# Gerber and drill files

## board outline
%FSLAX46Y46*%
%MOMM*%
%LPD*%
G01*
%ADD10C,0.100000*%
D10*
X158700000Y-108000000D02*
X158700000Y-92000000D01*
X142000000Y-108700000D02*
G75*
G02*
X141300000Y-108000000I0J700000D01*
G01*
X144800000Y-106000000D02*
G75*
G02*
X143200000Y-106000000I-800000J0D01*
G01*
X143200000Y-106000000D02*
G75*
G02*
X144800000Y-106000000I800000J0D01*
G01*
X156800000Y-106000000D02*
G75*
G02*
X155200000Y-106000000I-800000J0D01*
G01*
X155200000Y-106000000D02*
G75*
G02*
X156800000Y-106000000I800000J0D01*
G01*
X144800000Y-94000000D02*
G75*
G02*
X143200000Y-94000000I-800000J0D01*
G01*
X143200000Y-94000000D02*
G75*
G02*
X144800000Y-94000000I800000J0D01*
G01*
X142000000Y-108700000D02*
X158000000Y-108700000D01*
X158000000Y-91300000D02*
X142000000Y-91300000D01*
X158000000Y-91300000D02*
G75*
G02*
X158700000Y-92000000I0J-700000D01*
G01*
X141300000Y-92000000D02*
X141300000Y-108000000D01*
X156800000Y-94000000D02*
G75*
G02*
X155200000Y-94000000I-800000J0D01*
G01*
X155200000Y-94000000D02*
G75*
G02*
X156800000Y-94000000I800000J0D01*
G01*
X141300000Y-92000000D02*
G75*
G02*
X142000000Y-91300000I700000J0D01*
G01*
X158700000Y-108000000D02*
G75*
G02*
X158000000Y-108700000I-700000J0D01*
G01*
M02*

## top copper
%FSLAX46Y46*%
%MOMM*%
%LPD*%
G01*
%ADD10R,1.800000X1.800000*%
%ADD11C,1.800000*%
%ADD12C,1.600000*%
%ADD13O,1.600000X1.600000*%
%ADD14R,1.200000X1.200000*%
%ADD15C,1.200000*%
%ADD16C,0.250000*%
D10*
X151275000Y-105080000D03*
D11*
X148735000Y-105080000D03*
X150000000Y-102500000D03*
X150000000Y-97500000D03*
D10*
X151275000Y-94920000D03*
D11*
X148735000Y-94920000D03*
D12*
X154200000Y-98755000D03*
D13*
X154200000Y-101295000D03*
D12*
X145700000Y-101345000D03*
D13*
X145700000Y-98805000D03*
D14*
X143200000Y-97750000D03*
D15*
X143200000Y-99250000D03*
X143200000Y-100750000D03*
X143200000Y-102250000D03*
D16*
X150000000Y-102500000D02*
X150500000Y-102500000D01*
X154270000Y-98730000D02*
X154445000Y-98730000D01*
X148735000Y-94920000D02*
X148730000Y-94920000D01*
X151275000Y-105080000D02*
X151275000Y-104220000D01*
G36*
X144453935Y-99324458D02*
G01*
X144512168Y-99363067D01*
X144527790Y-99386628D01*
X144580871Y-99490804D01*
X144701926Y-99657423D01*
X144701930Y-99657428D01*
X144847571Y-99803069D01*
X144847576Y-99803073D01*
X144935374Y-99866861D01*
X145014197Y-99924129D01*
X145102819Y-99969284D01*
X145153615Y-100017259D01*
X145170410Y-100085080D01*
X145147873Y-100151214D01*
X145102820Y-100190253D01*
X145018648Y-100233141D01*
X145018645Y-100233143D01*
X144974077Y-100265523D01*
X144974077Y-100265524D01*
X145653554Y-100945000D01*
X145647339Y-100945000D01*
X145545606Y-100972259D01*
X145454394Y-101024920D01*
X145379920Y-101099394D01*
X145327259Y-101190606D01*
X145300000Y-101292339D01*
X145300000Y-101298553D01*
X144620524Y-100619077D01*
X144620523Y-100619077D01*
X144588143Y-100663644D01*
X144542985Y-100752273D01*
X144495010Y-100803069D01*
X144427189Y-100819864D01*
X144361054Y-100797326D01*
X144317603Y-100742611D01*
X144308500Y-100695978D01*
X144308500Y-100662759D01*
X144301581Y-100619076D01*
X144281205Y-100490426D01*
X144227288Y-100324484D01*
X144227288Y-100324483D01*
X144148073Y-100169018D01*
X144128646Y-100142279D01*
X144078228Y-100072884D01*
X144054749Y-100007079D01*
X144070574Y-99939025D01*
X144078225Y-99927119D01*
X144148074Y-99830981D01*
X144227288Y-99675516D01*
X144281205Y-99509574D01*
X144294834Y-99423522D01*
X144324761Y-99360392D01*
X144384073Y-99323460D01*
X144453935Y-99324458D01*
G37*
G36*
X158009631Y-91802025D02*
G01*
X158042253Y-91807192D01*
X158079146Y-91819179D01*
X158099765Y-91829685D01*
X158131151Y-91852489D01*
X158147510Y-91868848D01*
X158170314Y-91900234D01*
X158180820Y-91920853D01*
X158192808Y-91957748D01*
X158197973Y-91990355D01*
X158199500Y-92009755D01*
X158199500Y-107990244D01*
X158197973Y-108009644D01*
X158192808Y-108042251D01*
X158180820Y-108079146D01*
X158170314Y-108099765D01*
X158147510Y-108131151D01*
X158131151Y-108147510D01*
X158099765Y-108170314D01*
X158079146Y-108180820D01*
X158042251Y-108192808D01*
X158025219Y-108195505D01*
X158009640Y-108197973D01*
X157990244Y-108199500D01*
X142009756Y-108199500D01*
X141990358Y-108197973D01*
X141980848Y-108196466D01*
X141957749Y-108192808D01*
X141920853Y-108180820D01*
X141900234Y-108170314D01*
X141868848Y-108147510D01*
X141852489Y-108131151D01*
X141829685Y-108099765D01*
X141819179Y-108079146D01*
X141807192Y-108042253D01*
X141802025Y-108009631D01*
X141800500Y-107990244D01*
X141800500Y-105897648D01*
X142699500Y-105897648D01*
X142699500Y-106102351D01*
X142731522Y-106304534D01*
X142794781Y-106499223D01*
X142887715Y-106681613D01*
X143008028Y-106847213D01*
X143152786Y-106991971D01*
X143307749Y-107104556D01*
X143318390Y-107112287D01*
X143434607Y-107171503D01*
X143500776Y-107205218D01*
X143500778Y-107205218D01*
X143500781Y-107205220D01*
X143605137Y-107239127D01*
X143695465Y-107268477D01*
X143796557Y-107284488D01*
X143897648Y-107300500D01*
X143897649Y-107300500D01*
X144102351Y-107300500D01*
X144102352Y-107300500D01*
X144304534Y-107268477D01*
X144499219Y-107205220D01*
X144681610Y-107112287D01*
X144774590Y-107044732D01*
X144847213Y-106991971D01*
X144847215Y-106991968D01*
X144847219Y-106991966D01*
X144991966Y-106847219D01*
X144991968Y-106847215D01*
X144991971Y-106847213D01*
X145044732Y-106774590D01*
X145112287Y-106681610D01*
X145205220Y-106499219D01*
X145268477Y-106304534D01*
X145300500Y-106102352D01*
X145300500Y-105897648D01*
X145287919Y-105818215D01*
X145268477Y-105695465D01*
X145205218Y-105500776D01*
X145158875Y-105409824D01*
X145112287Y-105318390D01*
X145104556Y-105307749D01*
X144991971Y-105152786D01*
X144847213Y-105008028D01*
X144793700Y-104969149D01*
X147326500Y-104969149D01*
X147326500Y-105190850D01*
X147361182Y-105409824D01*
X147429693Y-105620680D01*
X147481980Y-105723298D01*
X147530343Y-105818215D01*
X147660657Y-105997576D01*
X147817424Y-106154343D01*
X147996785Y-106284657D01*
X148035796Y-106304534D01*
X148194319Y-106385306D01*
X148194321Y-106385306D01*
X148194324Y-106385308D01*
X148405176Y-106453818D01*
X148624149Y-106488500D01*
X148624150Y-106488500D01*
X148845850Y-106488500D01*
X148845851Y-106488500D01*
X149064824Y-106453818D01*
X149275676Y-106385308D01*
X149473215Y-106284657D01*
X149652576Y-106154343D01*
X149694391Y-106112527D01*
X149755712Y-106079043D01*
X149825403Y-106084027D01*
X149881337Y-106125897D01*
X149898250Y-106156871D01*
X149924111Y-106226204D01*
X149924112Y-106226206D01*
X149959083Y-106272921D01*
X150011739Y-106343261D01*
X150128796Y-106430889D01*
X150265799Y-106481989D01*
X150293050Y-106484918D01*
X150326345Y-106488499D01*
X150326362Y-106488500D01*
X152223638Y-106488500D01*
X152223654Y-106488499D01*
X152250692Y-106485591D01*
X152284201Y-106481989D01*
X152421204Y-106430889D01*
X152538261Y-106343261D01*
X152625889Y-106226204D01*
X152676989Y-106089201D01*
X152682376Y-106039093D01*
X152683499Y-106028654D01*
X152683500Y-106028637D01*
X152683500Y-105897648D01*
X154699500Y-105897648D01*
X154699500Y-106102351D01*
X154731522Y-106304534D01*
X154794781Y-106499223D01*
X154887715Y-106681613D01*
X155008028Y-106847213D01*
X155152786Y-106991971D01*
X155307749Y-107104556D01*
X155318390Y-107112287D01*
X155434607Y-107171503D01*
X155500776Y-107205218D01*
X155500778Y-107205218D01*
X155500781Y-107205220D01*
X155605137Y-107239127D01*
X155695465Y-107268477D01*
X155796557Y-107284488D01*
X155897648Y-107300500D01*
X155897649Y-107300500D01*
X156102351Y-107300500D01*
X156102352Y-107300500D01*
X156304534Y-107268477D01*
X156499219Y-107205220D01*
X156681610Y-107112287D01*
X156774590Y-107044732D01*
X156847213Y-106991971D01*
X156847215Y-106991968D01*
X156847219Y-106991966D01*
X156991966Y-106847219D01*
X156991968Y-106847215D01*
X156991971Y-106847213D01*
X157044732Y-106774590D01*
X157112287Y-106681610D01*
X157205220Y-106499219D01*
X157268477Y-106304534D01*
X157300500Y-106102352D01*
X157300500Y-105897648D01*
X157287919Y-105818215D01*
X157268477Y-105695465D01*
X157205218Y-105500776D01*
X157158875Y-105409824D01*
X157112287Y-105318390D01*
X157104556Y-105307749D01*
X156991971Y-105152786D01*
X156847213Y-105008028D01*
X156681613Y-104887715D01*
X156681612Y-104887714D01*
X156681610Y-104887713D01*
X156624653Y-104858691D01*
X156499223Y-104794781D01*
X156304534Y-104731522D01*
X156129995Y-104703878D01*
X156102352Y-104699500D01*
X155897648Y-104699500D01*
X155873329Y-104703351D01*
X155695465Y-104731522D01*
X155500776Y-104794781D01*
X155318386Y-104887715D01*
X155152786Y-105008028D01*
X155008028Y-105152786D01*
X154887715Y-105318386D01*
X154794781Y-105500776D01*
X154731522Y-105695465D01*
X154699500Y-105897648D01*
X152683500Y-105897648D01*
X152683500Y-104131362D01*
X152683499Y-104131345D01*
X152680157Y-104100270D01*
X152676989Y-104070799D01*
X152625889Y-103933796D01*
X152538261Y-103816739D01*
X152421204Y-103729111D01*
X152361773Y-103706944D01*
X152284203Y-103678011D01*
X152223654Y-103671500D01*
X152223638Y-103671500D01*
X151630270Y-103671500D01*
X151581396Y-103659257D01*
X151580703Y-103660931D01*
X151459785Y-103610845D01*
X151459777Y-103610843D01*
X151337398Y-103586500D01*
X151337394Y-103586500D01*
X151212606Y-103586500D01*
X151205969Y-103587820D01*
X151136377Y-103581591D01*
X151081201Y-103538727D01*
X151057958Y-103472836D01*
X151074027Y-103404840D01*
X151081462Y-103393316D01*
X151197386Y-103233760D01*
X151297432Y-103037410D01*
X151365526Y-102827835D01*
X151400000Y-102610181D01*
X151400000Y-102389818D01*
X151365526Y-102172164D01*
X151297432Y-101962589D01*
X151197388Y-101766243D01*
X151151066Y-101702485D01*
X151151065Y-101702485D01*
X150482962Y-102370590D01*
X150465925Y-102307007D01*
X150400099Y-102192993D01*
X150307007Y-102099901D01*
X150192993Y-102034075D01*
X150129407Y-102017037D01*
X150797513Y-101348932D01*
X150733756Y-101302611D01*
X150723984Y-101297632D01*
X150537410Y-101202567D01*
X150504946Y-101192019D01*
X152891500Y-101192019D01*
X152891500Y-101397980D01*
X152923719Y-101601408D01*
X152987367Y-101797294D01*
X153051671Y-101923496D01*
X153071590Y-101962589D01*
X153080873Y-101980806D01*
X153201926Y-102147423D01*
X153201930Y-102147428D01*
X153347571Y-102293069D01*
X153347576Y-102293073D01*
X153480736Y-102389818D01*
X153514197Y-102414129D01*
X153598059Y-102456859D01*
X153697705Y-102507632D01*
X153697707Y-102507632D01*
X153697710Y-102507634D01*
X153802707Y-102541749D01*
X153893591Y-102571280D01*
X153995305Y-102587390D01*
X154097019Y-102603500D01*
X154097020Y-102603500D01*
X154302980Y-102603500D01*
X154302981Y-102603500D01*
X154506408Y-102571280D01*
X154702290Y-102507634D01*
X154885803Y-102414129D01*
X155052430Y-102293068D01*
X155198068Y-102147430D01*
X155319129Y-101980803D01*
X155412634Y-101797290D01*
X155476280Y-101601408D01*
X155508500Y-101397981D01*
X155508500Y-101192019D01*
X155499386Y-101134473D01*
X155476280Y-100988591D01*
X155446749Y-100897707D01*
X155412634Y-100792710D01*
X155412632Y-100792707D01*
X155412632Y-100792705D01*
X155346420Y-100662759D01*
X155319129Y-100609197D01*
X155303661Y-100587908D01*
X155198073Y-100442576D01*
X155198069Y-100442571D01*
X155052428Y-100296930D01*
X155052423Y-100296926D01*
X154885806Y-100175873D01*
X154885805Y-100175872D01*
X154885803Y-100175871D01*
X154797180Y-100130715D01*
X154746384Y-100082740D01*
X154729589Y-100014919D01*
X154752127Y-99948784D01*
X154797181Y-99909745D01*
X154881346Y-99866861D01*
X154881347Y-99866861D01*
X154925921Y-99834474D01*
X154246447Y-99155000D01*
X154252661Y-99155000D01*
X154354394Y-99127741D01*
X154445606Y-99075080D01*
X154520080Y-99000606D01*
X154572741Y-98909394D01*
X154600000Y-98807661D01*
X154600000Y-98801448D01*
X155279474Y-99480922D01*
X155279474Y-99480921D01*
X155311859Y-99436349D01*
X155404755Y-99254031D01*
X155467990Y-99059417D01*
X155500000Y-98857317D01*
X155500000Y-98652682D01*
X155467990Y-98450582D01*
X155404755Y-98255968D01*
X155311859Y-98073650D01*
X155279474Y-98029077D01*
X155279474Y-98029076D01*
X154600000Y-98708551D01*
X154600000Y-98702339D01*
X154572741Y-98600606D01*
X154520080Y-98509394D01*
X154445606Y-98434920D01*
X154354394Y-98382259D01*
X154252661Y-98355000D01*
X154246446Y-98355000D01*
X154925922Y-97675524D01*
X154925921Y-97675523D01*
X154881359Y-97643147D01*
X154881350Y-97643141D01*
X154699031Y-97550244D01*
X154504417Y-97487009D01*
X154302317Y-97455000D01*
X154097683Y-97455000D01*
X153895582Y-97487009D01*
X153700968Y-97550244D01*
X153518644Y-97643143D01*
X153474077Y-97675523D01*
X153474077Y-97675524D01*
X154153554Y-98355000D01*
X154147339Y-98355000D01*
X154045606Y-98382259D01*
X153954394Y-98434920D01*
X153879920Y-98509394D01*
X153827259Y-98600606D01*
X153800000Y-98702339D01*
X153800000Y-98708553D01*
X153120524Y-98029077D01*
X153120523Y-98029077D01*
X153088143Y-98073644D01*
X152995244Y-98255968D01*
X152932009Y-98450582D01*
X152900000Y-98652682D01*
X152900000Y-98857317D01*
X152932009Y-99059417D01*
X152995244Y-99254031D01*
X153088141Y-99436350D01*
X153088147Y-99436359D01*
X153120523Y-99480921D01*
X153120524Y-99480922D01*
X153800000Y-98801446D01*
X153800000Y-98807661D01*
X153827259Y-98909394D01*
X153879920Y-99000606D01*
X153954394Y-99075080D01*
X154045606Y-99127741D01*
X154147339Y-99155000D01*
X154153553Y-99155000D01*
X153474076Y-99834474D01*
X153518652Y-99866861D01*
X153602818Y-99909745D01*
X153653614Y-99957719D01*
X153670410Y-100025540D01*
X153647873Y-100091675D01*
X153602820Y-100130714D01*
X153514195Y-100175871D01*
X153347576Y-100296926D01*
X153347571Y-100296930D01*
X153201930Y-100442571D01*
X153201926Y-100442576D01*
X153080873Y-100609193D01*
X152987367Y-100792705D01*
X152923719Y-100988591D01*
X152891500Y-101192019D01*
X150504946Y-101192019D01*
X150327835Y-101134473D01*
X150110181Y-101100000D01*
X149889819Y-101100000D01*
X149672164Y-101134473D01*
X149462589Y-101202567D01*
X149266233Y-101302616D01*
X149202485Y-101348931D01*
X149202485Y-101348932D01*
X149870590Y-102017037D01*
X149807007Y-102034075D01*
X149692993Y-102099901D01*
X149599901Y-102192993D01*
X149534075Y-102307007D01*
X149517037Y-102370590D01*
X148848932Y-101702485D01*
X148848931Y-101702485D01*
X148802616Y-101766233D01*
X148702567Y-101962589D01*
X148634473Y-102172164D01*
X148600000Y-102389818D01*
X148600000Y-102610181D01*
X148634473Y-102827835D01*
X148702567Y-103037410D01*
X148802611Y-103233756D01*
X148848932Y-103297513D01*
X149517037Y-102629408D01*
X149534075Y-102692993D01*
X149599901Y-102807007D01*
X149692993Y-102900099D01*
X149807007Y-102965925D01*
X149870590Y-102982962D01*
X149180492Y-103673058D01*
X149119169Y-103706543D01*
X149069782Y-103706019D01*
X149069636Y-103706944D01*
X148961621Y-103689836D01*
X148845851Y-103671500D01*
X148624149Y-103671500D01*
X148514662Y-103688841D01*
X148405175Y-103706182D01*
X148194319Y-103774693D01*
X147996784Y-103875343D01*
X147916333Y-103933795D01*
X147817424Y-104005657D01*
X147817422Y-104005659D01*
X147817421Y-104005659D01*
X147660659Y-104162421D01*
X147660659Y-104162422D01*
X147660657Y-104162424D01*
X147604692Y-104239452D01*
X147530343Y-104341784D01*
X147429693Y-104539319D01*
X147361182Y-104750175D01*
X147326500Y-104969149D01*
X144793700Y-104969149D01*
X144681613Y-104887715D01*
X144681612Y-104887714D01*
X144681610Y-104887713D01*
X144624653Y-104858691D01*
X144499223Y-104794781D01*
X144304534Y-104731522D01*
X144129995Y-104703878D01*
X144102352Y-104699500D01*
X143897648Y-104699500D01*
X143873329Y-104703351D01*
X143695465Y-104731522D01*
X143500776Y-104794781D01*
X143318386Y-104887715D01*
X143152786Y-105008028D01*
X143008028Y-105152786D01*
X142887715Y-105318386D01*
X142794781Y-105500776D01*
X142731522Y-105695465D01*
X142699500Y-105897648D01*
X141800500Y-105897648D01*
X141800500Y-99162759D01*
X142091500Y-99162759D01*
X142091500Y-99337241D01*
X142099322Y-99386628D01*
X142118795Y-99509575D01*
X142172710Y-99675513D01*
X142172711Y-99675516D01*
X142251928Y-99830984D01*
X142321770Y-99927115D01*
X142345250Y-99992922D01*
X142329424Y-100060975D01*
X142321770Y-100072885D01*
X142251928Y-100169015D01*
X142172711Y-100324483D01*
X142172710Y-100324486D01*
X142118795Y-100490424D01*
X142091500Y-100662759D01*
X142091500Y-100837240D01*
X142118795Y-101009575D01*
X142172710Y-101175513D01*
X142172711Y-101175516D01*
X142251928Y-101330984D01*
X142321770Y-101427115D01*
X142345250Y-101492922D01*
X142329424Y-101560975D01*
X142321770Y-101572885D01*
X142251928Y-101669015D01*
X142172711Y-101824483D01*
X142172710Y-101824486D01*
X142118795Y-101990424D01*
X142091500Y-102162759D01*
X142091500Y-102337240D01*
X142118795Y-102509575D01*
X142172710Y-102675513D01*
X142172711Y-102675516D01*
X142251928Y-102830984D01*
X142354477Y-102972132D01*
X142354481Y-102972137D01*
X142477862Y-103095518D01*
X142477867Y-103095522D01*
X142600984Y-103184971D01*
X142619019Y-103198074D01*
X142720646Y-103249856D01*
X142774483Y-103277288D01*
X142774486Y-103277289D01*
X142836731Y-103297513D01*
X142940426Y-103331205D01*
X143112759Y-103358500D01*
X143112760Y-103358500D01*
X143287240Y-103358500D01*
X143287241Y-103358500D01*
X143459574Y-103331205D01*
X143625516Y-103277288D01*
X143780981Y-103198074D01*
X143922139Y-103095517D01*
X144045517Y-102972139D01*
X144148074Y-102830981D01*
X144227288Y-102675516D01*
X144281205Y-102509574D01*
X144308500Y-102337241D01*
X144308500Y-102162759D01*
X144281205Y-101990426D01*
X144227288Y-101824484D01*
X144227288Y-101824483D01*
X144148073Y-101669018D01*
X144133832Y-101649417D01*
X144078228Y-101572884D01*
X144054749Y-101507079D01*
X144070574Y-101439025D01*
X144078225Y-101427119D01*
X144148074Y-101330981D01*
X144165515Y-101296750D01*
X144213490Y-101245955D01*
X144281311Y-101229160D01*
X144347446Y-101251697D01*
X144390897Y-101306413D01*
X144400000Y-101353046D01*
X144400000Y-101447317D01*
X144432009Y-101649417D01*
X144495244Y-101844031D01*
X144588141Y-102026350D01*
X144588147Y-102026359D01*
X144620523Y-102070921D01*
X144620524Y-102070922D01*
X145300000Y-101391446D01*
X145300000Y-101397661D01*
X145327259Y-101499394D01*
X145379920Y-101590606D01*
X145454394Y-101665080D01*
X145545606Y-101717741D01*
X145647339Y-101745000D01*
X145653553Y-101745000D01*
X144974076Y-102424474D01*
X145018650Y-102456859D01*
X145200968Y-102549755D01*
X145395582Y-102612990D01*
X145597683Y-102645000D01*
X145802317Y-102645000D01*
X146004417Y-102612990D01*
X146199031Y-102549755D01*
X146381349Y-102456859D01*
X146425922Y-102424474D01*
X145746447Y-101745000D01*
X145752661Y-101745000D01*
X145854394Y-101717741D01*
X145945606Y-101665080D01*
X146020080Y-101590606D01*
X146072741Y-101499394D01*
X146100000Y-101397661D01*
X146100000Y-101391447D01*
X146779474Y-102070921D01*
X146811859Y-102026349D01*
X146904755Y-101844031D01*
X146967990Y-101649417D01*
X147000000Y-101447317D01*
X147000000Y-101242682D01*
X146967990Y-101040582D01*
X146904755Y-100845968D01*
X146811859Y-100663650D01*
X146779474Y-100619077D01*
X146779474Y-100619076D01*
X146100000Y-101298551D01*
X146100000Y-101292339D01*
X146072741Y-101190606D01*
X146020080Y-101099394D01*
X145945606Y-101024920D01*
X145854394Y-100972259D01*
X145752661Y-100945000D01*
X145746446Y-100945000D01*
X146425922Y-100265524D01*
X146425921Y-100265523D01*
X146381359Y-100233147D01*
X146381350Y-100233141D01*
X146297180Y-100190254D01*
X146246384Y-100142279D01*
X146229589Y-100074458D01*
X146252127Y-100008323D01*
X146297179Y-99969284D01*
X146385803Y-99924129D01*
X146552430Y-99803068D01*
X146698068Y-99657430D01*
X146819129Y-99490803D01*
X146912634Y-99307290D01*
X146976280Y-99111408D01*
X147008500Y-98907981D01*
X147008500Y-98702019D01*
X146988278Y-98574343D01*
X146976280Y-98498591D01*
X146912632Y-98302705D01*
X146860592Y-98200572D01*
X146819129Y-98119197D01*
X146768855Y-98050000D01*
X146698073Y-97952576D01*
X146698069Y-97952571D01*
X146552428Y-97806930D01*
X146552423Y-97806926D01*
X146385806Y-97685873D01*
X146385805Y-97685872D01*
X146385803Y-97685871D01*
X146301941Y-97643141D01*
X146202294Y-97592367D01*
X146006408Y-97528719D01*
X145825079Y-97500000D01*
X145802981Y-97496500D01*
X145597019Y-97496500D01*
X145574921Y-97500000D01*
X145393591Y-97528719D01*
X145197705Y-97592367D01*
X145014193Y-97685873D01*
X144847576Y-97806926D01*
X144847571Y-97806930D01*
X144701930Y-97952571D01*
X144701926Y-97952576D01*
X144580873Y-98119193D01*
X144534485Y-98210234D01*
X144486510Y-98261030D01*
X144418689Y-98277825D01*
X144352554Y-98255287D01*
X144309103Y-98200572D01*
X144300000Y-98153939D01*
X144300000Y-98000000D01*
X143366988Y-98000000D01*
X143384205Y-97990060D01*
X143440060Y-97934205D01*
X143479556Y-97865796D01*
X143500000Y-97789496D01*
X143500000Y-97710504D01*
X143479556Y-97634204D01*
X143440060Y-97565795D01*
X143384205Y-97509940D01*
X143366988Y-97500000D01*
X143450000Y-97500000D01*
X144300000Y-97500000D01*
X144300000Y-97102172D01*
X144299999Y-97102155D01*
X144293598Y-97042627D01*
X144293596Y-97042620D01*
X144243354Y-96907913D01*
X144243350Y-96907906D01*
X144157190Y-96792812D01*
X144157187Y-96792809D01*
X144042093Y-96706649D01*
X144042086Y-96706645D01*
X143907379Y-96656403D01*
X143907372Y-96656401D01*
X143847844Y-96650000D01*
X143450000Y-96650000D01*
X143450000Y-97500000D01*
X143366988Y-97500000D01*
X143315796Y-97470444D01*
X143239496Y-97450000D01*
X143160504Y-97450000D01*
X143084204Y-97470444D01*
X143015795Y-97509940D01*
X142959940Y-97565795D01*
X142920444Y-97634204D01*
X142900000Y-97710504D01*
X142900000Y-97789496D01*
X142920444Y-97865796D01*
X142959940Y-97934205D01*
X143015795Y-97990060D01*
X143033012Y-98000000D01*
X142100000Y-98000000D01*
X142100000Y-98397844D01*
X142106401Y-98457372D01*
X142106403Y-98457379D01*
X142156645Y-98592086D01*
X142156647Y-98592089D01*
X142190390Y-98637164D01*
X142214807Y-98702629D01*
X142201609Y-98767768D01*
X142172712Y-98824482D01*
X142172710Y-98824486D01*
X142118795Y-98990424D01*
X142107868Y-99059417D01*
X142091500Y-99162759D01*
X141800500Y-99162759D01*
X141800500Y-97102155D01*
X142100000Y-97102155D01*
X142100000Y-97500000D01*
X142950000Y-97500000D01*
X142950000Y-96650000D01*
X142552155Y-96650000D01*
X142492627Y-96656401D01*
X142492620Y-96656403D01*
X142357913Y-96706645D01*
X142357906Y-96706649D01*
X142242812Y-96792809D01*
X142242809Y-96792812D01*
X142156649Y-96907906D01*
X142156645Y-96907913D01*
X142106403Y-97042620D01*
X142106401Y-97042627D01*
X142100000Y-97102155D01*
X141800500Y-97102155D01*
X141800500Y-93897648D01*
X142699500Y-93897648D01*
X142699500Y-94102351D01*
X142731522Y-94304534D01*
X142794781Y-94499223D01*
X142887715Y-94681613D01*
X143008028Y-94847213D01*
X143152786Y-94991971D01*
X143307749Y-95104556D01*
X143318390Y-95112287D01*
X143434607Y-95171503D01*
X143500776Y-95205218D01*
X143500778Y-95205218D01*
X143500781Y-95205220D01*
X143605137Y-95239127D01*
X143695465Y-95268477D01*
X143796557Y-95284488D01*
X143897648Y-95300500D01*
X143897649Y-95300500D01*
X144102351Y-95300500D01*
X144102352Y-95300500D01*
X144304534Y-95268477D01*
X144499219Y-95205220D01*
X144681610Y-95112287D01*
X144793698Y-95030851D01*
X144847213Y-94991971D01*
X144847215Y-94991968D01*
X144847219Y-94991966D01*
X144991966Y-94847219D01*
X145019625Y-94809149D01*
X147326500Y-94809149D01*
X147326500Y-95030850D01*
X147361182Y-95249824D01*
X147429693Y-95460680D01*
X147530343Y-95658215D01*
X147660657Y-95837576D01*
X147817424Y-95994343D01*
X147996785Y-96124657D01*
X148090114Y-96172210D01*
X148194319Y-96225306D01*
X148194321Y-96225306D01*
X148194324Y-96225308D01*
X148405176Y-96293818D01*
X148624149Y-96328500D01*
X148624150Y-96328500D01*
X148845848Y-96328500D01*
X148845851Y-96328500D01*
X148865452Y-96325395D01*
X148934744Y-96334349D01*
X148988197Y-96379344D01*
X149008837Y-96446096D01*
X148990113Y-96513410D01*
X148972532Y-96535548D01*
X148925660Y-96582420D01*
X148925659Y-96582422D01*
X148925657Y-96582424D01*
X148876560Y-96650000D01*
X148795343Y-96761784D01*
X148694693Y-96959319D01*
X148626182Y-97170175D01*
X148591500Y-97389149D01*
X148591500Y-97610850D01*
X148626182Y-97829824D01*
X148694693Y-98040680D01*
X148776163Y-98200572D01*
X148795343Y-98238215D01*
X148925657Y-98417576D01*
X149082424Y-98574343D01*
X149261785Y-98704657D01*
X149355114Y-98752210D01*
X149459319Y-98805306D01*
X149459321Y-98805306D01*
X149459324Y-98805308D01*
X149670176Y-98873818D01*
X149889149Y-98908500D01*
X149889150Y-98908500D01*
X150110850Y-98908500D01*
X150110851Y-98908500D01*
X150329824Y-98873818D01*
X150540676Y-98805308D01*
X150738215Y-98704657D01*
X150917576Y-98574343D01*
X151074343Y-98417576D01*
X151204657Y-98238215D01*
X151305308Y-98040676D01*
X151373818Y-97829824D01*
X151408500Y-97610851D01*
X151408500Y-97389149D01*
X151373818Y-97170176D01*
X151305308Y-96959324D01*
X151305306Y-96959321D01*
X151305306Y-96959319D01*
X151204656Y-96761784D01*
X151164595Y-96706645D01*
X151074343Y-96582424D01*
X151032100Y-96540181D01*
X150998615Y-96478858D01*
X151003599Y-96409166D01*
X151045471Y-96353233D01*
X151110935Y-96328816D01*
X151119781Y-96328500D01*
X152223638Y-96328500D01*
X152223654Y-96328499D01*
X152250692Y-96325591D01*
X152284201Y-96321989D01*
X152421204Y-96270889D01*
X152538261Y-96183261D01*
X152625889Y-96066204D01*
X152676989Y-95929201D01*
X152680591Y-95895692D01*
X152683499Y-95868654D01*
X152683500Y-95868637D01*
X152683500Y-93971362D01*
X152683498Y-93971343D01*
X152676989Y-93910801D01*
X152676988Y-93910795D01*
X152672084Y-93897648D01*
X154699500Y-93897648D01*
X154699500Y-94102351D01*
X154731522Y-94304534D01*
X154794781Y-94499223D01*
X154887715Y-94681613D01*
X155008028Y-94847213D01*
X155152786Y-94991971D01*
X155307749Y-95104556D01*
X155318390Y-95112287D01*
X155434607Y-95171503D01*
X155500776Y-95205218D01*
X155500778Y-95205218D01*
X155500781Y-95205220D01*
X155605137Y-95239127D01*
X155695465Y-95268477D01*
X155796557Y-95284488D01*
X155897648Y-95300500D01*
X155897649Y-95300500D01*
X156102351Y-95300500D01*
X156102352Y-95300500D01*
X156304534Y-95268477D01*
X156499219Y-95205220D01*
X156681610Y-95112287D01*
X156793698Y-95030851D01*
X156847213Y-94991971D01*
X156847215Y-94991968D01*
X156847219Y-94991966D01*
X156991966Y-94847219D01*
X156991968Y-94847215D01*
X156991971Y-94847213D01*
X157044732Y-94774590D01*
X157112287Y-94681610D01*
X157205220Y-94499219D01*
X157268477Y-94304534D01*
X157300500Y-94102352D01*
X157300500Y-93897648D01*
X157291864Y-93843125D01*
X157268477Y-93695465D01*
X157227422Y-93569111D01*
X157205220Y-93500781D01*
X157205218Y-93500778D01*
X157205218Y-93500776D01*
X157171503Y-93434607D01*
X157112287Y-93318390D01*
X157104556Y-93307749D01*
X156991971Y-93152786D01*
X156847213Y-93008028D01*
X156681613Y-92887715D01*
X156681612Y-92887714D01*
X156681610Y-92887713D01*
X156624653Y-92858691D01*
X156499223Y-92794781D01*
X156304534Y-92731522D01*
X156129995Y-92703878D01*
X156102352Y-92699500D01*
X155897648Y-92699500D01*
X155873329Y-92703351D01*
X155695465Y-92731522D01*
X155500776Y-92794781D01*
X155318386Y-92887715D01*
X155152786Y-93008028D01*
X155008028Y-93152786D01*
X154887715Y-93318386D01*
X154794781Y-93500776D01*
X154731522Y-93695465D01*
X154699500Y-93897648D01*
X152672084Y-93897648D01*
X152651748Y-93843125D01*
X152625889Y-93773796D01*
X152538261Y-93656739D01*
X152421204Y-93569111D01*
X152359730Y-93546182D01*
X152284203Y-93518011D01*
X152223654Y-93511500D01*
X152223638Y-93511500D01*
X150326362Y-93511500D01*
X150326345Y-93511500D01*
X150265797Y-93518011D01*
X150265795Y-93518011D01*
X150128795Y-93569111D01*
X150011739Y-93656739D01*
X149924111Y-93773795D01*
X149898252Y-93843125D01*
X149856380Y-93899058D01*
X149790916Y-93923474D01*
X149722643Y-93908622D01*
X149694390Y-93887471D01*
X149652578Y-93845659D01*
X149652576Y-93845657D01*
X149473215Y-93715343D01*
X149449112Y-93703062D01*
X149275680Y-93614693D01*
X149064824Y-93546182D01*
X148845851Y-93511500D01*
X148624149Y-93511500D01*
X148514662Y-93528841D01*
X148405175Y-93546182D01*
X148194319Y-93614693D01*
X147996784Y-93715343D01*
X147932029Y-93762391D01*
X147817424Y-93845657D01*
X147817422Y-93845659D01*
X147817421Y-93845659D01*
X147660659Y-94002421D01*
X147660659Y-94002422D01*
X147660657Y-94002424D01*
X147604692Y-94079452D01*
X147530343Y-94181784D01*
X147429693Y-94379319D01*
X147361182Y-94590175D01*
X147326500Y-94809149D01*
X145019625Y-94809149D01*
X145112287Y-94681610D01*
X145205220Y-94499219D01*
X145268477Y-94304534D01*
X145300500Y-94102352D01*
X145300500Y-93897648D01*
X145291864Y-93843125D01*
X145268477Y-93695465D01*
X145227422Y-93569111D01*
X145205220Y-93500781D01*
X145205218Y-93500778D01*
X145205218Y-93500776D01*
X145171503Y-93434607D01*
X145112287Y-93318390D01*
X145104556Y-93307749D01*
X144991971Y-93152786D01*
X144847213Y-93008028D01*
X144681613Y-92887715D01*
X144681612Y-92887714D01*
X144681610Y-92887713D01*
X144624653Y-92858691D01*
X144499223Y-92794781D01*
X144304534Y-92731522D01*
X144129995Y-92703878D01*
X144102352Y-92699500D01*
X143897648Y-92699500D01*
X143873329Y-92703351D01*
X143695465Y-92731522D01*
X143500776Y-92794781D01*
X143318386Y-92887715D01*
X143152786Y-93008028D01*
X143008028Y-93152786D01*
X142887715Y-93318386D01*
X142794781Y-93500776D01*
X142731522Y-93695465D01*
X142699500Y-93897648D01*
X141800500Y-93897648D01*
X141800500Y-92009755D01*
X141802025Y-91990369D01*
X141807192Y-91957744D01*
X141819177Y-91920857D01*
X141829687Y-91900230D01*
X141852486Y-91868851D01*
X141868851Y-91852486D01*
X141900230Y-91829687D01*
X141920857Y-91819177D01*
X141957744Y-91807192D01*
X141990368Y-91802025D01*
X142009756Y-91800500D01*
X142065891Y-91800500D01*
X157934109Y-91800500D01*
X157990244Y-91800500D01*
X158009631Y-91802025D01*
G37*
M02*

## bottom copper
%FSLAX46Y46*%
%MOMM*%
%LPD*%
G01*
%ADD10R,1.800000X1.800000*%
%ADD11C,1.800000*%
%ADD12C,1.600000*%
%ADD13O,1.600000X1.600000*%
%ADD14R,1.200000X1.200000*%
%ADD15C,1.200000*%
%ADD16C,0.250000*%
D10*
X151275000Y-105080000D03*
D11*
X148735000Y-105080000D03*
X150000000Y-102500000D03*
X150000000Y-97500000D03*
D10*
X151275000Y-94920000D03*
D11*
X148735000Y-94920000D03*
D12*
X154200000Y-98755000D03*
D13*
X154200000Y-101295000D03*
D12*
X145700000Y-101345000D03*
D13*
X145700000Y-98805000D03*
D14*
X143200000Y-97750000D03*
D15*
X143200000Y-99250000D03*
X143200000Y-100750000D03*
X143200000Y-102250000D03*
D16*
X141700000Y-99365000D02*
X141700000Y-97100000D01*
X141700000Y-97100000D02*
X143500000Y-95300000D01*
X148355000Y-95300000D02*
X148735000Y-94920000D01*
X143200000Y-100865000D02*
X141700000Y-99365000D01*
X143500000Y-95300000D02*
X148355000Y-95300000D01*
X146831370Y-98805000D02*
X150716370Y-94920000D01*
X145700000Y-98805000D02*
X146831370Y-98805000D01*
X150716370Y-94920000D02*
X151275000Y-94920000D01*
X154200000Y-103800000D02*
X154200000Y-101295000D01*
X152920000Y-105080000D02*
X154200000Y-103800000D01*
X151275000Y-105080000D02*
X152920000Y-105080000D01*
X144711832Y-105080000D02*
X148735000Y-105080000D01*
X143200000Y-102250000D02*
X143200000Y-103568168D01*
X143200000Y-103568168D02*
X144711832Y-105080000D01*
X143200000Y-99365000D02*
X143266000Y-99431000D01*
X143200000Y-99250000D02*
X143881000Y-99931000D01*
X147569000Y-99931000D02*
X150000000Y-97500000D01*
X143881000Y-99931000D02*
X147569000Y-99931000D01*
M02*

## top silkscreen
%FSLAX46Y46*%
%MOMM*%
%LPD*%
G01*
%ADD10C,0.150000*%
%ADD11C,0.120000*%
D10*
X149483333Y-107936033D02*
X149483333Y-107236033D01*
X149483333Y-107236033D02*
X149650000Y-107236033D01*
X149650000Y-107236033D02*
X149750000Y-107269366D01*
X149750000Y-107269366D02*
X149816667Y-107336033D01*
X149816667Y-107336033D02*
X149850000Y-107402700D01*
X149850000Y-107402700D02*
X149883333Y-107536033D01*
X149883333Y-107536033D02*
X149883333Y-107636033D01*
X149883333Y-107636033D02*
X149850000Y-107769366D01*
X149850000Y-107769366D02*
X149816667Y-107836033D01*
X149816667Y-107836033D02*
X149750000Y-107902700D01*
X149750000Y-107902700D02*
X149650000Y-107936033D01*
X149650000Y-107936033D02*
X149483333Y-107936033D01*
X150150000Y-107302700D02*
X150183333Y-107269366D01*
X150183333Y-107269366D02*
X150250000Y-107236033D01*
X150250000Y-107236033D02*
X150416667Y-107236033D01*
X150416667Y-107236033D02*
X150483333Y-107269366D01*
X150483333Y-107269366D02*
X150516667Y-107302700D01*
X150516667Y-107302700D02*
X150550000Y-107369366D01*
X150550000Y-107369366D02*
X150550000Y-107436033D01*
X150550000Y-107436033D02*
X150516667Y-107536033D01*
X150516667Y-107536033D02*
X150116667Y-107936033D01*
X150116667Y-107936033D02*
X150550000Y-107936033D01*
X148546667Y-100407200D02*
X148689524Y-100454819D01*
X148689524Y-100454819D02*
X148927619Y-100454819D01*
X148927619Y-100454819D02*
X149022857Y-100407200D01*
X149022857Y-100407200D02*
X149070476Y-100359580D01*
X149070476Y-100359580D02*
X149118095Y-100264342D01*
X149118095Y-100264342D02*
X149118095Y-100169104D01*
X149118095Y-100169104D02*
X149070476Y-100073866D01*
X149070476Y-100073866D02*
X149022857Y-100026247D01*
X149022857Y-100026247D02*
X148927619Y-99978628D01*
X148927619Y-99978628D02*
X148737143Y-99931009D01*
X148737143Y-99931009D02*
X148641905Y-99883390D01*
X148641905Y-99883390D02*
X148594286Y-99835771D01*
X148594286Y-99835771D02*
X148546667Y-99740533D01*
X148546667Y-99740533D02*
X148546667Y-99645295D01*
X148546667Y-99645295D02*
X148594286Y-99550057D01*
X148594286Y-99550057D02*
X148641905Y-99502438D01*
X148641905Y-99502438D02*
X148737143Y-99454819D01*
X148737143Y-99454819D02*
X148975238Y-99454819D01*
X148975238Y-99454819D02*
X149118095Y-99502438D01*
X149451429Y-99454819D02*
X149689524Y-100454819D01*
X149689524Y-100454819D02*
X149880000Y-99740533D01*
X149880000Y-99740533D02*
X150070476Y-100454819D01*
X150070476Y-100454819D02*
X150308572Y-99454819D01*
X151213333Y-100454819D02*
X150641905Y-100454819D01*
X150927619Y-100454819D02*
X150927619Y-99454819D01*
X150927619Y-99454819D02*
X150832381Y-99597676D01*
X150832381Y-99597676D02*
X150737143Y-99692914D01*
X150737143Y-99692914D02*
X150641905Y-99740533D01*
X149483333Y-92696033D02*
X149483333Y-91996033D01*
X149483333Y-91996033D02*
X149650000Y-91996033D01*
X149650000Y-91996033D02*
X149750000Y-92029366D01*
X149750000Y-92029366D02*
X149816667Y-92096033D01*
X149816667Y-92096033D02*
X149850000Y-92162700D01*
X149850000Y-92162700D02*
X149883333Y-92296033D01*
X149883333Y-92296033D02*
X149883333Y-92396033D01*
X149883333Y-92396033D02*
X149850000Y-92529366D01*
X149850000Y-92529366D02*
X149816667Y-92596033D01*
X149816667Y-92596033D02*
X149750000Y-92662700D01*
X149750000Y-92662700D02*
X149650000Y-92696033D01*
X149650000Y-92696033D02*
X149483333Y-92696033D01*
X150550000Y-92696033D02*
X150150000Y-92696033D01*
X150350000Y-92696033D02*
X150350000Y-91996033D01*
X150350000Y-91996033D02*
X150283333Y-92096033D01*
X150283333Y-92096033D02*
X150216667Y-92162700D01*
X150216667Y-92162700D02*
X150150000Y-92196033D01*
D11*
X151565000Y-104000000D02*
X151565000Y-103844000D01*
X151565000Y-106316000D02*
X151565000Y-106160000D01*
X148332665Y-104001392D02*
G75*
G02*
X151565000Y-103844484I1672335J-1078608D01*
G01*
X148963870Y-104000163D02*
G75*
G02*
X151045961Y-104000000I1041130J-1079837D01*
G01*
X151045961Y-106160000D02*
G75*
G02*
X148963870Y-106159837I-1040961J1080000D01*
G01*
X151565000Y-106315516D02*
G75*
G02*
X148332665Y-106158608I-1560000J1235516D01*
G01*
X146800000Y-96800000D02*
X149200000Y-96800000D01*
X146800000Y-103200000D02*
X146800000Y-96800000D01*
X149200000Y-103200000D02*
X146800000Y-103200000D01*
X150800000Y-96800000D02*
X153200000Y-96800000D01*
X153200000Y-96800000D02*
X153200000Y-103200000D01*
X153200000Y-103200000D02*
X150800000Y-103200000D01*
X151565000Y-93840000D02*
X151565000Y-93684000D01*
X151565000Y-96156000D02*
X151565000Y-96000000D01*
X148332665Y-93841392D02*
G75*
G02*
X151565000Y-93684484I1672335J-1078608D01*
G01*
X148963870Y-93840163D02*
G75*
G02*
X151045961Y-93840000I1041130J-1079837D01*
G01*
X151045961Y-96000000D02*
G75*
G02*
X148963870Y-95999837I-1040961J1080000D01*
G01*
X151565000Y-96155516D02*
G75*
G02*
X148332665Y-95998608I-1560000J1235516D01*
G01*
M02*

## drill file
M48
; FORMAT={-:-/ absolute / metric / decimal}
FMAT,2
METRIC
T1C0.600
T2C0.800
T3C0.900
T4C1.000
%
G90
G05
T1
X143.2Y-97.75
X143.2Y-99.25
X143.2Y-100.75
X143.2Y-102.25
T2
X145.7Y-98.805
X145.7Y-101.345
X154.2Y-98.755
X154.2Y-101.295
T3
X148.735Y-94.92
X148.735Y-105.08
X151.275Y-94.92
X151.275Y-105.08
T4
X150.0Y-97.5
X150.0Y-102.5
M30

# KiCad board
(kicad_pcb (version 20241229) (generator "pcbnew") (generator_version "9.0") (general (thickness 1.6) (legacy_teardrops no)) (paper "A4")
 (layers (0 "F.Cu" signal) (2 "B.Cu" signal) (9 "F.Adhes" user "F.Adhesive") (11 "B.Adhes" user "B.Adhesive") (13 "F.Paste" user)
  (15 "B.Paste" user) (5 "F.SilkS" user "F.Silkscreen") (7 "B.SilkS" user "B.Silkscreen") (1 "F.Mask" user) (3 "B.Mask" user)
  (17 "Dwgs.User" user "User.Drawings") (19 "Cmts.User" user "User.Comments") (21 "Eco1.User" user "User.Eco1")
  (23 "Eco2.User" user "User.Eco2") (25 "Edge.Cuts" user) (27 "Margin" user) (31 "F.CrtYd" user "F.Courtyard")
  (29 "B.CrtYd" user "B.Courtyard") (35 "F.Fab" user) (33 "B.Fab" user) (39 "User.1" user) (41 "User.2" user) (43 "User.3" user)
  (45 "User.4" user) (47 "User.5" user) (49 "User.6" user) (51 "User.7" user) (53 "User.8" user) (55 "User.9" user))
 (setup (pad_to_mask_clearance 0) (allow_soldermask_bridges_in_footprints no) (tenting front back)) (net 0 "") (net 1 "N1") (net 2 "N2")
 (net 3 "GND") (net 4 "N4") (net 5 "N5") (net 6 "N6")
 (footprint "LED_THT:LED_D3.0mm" (layer "F.Cu") (at 151.275 105.08 180)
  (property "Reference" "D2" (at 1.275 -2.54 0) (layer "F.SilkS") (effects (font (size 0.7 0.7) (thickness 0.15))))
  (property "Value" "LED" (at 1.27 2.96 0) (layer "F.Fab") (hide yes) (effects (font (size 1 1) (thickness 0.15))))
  (fp_line (start -0.29 1.08) (end -0.29 1.236) (stroke (width 0.12) (type solid)) (layer "F.SilkS"))
  (fp_line (start -0.29 -1.236) (end -0.29 -1.08) (stroke (width 0.12) (type solid)) (layer "F.SilkS"))
  (fp_arc (start 2.942335 1.078608) (mid 1.366487 1.987659) (end -0.29 1.235516) (stroke (width 0.12) (type solid)) (layer "F.SilkS"))
  (fp_arc (start 2.31113 1.079837) (mid 1.270117 1.5) (end 0.229039 1.08) (stroke (width 0.12) (type solid)) (layer "F.SilkS"))
  (fp_arc (start 0.229039 -1.08) (mid 1.270117 -1.5) (end 2.31113 -1.079837) (stroke (width 0.12) (type solid)) (layer "F.SilkS"))
  (fp_arc (start -0.29 -1.235516) (mid 1.366487 -1.987659) (end 2.942335 -1.078608) (stroke (width 0.12) (type solid)) (layer "F.SilkS"))
  (pad "1" thru_hole rect (at 0 0 180) (size 1.8 1.8) (drill 0.9) (layers "*.Cu" "*.Mask") (remove_unused_layers no) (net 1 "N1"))
  (pad "2" thru_hole circle (at 2.54 0 180) (size 1.8 1.8) (drill 0.9) (layers "*.Cu" "*.Mask") (remove_unused_layers no) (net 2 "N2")))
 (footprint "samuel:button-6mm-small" (layer "F.Cu") (at 150 100 90)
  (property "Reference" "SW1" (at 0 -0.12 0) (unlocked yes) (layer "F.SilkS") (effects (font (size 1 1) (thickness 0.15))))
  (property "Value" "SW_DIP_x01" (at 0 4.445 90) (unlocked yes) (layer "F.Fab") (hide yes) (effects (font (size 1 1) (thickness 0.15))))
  (fp_line (start 3.2 -3.2) (end 3.2 -0.8) (stroke (width 0.12) (type solid)) (layer "F.SilkS"))
  (fp_line (start -3.2 -3.2) (end 3.2 -3.2) (stroke (width 0.12) (type solid)) (layer "F.SilkS"))
  (fp_line (start -3.2 -0.8) (end -3.2 -3.2) (stroke (width 0.12) (type solid)) (layer "F.SilkS"))
  (fp_line (start 3.2 0.8) (end 3.2 3.2) (stroke (width 0.12) (type solid)) (layer "F.SilkS"))
  (fp_line (start 3.2 3.2) (end -3.2 3.2) (stroke (width 0.12) (type solid)) (layer "F.SilkS"))
  (fp_line (start -3.2 3.2) (end -3.2 0.8) (stroke (width 0.12) (type solid)) (layer "F.SilkS"))
  (pad "1" thru_hole circle (at -2.5 0 90) (size 1.8 1.8) (drill 1) (layers "*.Cu" "*.Mask") (remove_unused_layers no) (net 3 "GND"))
  (pad "2" thru_hole circle (at 2.5 0 90) (size 1.8 1.8) (drill 1) (layers "*.Cu" "*.Mask") (remove_unused_layers no) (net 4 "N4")))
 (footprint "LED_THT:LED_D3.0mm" (layer "F.Cu") (at 151.275 94.92 180)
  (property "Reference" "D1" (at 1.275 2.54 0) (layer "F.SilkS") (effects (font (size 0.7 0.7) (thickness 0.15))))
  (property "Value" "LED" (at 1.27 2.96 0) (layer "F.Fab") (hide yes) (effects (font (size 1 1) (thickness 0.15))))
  (fp_line (start -0.29 1.08) (end -0.29 1.236) (stroke (width 0.12) (type solid)) (layer "F.SilkS"))
  (fp_line (start -0.29 -1.236) (end -0.29 -1.08) (stroke (width 0.12) (type solid)) (layer "F.SilkS"))
  (fp_arc (start 2.942335 1.078608) (mid 1.366487 1.987659) (end -0.29 1.235516) (stroke (width 0.12) (type solid)) (layer "F.SilkS"))
  (fp_arc (start 2.31113 1.079837) (mid 1.270117 1.5) (end 0.229039 1.08) (stroke (width 0.12) (type solid)) (layer "F.SilkS"))
  (fp_arc (start 0.229039 -1.08) (mid 1.270117 -1.5) (end 2.31113 -1.079837) (stroke (width 0.12) (type solid)) (layer "F.SilkS"))
  (fp_arc (start -0.29 -1.235516) (mid 1.366487 -1.987659) (end 2.942335 -1.078608) (stroke (width 0.12) (type solid)) (layer "F.SilkS"))
  (pad "1" thru_hole rect (at 0 0 180) (size 1.8 1.8) (drill 0.9) (layers "*.Cu" "*.Mask") (remove_unused_layers no) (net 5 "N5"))
  (pad "2" thru_hole circle (at 2.54 0 180) (size 1.8 1.8) (drill 0.9) (layers "*.Cu" "*.Mask") (remove_unused_layers no) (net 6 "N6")))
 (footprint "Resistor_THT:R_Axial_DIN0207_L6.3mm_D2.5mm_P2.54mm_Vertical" (layer "B.Cu") (at 154.2 98.755 -90)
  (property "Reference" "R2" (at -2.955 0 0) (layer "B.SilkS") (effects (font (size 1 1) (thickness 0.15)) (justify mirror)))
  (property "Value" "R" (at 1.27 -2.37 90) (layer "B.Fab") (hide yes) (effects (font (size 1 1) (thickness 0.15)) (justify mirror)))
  (pad "1" thru_hole circle (at 0 0 270) (size 1.6 1.6) (drill 0.8) (layers "*.Cu" "*.Mask") (remove_unused_layers no) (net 3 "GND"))
  (pad "2" thru_hole oval (at 2.54 0 270) (size 1.6 1.6) (drill 0.8) (layers "*.Cu" "*.Mask") (remove_unused_layers no) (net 1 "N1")))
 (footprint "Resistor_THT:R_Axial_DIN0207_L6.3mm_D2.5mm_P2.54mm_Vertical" (layer "B.Cu") (at 145.7 101.345 90)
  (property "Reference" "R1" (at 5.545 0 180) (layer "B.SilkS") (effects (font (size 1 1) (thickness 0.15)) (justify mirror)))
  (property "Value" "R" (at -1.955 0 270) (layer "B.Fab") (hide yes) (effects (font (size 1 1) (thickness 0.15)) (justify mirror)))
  (pad "1" thru_hole circle (at 0 0 90) (size 1.6 1.6) (drill 0.8) (layers "*.Cu" "*.Mask") (remove_unused_layers no) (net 3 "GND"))
  (pad "2" thru_hole oval (at 2.54 0 90) (size 1.6 1.6) (drill 0.8) (layers "*.Cu" "*.Mask") (remove_unused_layers no) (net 5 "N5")))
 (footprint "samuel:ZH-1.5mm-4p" (layer "B.Cu") (at 143.2 100 180)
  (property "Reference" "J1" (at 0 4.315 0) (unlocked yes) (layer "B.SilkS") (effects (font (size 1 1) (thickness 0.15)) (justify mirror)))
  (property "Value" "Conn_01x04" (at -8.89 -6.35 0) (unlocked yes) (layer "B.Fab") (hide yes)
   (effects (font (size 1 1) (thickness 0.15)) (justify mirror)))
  (pad "1" thru_hole rect (at 0 2.25 180) (size 1.2 1.2) (drill 0.6) (layers "*.Cu" "*.Mask") (remove_unused_layers no) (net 3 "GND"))
  (pad "2" thru_hole circle (at 0 0.75 180) (size 1.2 1.2) (drill 0.6) (layers "*.Cu" "*.Mask") (remove_unused_layers no) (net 4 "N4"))
  (pad "3" thru_hole circle (at 0 -0.75 180) (size 1.2 1.2) (drill 0.6) (layers "*.Cu" "*.Mask") (remove_unused_layers no) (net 6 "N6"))
  (pad "4" thru_hole circle (at 0 -2.25 180) (size 1.2 1.2) (drill 0.6) (layers "*.Cu" "*.Mask") (remove_unused_layers no) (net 2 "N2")))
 (gr_line (start 158.7 108) (end 158.7 92) (stroke (width 0.1) (type solid)) (layer "Edge.Cuts"))
 (gr_arc (start 142 108.7) (mid 141.505025 108.494975) (end 141.3 108) (stroke (width 0.1) (type solid)) (layer "Edge.Cuts"))
 (gr_circle (center 144 106) (end 144.8 106) (stroke (width 0.1) (type solid)) (fill no) (layer "Edge.Cuts"))
 (gr_circle (center 156 106) (end 155.2 106) (stroke (width 0.1) (type solid)) (fill no) (layer "Edge.Cuts"))
 (gr_circle (center 144 94) (end 144.8 94) (stroke (width 0.1) (type solid)) (fill no) (layer "Edge.Cuts"))
 (gr_line (start 142 108.7) (end 158 108.7) (stroke (width 0.1) (type solid)) (layer "Edge.Cuts"))
 (gr_line (start 158 91.3) (end 142 91.3) (stroke (width 0.1) (type solid)) (layer "Edge.Cuts"))
 (gr_arc (start 158 91.3) (mid 158.494975 91.505025) (end 158.7 92) (stroke (width 0.1) (type solid)) (layer "Edge.Cuts"))
 (gr_line (start 141.3 92) (end 141.3 108) (stroke (width 0.1) (type solid)) (layer "Edge.Cuts"))
 (gr_circle (center 156 94) (end 156 94.8) (stroke (width 0.1) (type solid)) (fill no) (layer "Edge.Cuts"))
 (gr_arc (start 141.3 92) (mid 141.505025 91.505025) (end 142 91.3) (stroke (width 0.1) (type solid)) (layer "Edge.Cuts"))
 (gr_arc (start 158.7 108) (mid 158.494975 108.494975) (end 158 108.7) (stroke (width 0.1) (type solid)) (layer "Edge.Cuts"))
 (segment (start 150 102.5) (end 150.5 102.5) (width 0.25) (layer "F.Cu") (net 3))
 (segment (start 154.27 98.73) (end 154.445 98.73) (width 0.25) (layer "F.Cu") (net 3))
 (segment (start 148.735 94.92) (end 148.73 94.92) (width 0.25) (layer "F.Cu") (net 6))
 (segment (start 141.7 99.365) (end 141.7 97.1) (width 0.25) (layer "B.Cu") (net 6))
 (segment (start 141.7 97.1) (end 143.5 95.3) (width 0.25) (layer "B.Cu") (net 6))
 (segment (start 148.355 95.3) (end 148.735 94.92) (width 0.25) (layer "B.Cu") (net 6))
 (segment (start 143.2 100.865) (end 141.7 99.365) (width 0.25) (layer "B.Cu") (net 6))
 (segment (start 143.5 95.3) (end 148.355 95.3) (width 0.25) (layer "B.Cu") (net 6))
 (segment (start 146.83137 98.805) (end 150.71637 94.92) (width 0.25) (layer "B.Cu") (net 5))
 (segment (start 145.7 98.805) (end 146.83137 98.805) (width 0.25) (layer "B.Cu") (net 5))
 (segment (start 150.71637 94.92) (end 151.275 94.92) (width 0.25) (layer "B.Cu") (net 5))
 (segment (start 151.275 105.08) (end 151.275 104.22) (width 0.25) (layer "F.Cu") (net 1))
 (segment (start 154.2 103.8) (end 154.2 101.295) (width 0.25) (layer "B.Cu") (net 1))
 (segment (start 152.92 105.08) (end 154.2 103.8) (width 0.25) (layer "B.Cu") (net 1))
 (segment (start 151.275 105.08) (end 152.92 105.08) (width 0.25) (layer "B.Cu") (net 1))
 (segment (start 144.711832 105.08) (end 148.735 105.08) (width 0.25) (layer "B.Cu") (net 2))
 (segment (start 143.2 102.25) (end 143.2 103.568168) (width 0.25) (layer "B.Cu") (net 2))
 (segment (start 143.2 103.568168) (end 144.711832 105.08) (width 0.25) (layer "B.Cu") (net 2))
 (segment (start 143.2 99.365) (end 143.266 99.431) (width 0.25) (layer "B.Cu") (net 4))
 (segment (start 143.2 99.25) (end 143.881 99.931) (width 0.25) (layer "B.Cu") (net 4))
 (segment (start 147.569 99.931) (end 150 97.5) (width 0.25) (layer "B.Cu") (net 4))
 (segment (start 143.881 99.931) (end 147.569 99.931) (width 0.25) (layer "B.Cu") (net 4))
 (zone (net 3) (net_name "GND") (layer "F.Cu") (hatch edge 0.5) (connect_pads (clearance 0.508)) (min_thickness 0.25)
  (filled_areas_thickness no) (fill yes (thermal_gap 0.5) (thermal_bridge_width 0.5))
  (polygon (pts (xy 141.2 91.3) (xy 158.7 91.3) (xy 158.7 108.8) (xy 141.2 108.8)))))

